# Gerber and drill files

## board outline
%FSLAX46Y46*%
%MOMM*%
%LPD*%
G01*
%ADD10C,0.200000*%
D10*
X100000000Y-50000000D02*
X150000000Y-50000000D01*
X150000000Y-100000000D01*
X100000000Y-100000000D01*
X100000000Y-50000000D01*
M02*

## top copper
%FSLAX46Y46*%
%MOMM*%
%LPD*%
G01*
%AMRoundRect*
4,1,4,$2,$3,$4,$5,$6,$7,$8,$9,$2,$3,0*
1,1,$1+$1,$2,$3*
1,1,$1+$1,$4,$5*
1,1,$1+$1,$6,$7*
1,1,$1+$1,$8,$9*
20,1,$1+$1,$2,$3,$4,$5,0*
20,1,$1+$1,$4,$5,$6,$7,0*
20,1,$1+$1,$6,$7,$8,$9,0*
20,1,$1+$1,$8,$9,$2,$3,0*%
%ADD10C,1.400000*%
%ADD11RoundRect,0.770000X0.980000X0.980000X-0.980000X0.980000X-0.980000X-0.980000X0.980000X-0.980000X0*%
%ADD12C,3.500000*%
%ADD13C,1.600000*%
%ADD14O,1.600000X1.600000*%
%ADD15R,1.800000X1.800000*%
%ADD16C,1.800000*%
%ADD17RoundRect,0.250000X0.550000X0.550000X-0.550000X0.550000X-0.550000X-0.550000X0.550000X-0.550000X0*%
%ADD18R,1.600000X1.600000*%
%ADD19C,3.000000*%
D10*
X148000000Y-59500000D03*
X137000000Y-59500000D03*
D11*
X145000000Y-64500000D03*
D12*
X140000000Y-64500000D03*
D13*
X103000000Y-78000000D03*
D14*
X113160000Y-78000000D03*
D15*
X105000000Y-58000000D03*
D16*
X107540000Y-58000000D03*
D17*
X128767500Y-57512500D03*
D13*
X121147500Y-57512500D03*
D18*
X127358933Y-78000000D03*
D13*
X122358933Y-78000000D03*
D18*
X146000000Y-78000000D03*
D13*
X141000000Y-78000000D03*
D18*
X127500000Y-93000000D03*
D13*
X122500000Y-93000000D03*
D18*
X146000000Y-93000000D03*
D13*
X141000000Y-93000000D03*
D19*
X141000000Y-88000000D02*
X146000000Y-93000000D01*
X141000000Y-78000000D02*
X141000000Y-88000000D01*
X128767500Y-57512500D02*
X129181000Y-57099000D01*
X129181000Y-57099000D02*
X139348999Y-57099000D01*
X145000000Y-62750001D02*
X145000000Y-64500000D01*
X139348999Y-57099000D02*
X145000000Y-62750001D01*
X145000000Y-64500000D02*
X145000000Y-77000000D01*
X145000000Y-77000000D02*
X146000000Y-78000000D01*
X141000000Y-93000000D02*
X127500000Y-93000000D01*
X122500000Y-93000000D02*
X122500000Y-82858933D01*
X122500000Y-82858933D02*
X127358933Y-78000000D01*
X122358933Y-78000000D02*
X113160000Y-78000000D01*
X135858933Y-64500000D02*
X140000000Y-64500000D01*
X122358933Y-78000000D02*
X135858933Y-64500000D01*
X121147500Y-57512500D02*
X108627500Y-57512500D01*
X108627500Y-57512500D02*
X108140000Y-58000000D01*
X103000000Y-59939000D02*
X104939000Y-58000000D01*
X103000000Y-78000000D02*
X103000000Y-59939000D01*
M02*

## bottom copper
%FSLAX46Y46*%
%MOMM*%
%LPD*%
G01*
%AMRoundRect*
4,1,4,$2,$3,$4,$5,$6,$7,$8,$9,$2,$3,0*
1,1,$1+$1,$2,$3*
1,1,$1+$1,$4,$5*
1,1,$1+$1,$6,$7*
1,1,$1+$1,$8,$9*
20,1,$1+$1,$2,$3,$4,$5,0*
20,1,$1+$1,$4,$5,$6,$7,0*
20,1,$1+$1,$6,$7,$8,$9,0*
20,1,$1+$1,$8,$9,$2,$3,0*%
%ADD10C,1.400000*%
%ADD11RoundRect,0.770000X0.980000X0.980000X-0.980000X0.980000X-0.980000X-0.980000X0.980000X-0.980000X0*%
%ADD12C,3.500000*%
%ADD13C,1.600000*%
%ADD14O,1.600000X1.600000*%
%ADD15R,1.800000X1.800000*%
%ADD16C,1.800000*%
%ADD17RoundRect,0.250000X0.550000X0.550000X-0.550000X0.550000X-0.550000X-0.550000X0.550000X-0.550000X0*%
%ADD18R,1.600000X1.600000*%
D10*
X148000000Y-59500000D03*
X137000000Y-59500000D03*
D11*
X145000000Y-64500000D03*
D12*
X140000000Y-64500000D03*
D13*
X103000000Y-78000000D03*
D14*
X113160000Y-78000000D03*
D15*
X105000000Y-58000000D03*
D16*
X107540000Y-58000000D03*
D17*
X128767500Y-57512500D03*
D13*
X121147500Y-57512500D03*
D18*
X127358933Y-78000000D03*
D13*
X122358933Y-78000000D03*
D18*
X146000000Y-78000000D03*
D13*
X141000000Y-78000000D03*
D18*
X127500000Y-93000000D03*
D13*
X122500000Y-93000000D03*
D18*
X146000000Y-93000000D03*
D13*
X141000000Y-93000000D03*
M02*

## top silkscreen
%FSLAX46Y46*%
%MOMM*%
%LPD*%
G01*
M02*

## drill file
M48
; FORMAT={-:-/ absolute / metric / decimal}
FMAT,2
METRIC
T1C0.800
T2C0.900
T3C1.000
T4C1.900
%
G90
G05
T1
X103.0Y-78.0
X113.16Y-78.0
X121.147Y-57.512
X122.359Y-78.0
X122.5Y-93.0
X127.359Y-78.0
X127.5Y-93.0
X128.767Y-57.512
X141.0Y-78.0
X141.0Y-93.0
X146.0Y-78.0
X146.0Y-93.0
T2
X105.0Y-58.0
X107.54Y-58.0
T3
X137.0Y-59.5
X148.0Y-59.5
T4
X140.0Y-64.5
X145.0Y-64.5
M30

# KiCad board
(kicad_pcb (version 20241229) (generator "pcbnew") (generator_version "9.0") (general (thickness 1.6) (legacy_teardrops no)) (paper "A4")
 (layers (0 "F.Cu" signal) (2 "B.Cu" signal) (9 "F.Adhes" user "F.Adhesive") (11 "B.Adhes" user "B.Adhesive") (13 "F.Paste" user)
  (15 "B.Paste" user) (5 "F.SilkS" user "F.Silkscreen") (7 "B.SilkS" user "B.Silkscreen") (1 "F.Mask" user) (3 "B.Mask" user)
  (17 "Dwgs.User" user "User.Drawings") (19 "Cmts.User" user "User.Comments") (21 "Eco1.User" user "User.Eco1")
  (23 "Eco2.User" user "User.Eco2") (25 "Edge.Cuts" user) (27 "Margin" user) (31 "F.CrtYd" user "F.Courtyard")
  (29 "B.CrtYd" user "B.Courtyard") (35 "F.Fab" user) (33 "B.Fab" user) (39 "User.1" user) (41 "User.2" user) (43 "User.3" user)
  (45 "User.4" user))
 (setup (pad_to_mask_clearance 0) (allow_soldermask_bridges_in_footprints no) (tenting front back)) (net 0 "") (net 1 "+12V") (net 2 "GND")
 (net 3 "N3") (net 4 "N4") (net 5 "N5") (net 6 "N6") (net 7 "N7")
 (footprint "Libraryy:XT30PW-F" (layer "B.Cu") (at 145 64.5 180)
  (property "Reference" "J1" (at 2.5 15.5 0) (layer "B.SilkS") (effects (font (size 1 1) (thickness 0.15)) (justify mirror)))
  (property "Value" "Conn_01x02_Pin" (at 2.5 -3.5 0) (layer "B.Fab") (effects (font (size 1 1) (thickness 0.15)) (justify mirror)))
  (pad "" thru_hole circle (at -3 5 90) (size 1.4 1.4) (drill 1) (layers "*.Cu" "*.Mask") (remove_unused_layers no))
  (pad "" thru_hole circle (at 8 5 180) (size 1.4 1.4) (drill 1) (layers "*.Cu" "*.Mask") (remove_unused_layers no))
  (pad "1" thru_hole roundrect (at 0 0 180) (size 3.5 3.5) (drill 1.9) (layers "*.Cu" "*.Mask") (remove_unused_layers no)
   (roundrect_rratio 0.22) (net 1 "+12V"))
  (pad "2" thru_hole circle (at 5 0 180) (size 3.5 3.5) (drill 1.9) (layers "*.Cu" "*.Mask") (remove_unused_layers no) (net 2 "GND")))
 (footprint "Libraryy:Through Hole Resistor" (layer "B.Cu") (at 103 78)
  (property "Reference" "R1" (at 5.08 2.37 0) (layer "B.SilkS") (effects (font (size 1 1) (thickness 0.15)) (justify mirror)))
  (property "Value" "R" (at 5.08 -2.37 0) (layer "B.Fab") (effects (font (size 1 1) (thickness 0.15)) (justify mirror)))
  (pad "1" thru_hole circle (at 0 0) (size 1.6 1.6) (drill 0.8) (layers "*.Cu" "*.Mask") (remove_unused_layers no) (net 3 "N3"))
  (pad "2" thru_hole oval (at 10.16 0) (size 1.6 1.6) (drill 0.8) (layers "*.Cu" "*.Mask") (remove_unused_layers no) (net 2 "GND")))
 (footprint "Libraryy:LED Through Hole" (layer "B.Cu") (at 105 58)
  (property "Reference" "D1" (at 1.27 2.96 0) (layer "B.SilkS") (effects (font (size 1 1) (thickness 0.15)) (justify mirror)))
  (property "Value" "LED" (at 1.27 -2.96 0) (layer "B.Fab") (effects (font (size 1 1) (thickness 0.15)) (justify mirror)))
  (pad "1" thru_hole rect (at 0 0) (size 1.8 1.8) (drill 0.9) (layers "*.Cu" "*.Mask") (remove_unused_layers no) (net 3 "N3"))
  (pad "2" thru_hole circle (at 2.54 0) (size 1.8 1.8) (drill 0.9) (layers "*.Cu" "*.Mask") (remove_unused_layers no) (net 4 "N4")))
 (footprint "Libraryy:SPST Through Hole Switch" (layer "B.Cu") (at 128.7675 57.5125 180)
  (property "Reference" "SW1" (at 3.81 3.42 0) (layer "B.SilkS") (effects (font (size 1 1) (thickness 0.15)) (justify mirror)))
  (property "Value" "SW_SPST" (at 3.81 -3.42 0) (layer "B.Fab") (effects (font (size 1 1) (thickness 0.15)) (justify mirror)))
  (pad "1" thru_hole roundrect (at 0 0 180) (size 1.6 1.6) (drill 0.8) (layers "*.Cu" "*.Mask") (remove_unused_layers no)
   (roundrect_rratio 0.15625) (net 1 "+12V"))
  (pad "2" thru_hole circle (at 7.62 0 180) (size 1.6 1.6) (drill 0.8) (layers "*.Cu" "*.Mask") (remove_unused_layers no) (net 4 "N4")))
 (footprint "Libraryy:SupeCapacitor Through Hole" (layer "B.Cu") (at 127.358933 78 180)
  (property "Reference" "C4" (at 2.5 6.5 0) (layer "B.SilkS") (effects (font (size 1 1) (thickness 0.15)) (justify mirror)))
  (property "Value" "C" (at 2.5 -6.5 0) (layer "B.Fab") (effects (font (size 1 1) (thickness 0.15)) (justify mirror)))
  (pad "1" thru_hole rect (at 0 0 180) (size 1.6 1.6) (drill 0.8) (layers "*.Cu" "*.Mask") (remove_unused_layers no) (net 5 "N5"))
  (pad "2" thru_hole circle (at 5 0 180) (size 1.6 1.6) (drill 0.8) (layers "*.Cu" "*.Mask") (remove_unused_layers no) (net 2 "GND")))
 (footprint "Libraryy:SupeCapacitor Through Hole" (layer "B.Cu") (at 146 78 180)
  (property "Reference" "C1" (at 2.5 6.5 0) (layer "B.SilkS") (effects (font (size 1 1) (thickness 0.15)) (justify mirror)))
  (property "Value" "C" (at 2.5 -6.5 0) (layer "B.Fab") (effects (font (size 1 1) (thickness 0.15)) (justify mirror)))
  (pad "1" thru_hole rect (at 0 0 180) (size 1.6 1.6) (drill 0.8) (layers "*.Cu" "*.Mask") (remove_unused_layers no) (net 1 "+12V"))
  (pad "2" thru_hole circle (at 5 0 180) (size 1.6 1.6) (drill 0.8) (layers "*.Cu" "*.Mask") (remove_unused_layers no) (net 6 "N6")))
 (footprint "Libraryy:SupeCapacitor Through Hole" (layer "B.Cu") (at 127.5 93 180)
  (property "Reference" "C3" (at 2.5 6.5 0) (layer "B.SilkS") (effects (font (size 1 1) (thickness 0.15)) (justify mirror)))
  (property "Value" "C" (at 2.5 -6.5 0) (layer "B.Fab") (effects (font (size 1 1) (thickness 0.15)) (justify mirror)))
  (pad "1" thru_hole rect (at 0 0 180) (size 1.6 1.6) (drill 0.8) (layers "*.Cu" "*.Mask") (remove_unused_layers no) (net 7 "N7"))
  (pad "2" thru_hole circle (at 5 0 180) (size 1.6 1.6) (drill 0.8) (layers "*.Cu" "*.Mask") (remove_unused_layers no) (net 5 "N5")))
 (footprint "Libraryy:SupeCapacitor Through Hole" (layer "B.Cu") (at 146 93 180)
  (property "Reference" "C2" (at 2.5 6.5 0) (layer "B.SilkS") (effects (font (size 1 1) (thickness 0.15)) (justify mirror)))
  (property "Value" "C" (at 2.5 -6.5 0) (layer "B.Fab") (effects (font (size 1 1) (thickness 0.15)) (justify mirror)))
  (pad "1" thru_hole rect (at 0 0 180) (size 1.6 1.6) (drill 0.8) (layers "*.Cu" "*.Mask") (remove_unused_layers no) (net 6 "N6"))
  (pad "2" thru_hole circle (at 5 0 180) (size 1.6 1.6) (drill 0.8) (layers "*.Cu" "*.Mask") (remove_unused_layers no) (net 7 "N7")))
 (gr_rect (start 100 50) (end 150 100) (stroke (width 0.2) (type solid)) (fill no) (layer "Edge.Cuts"))
 (segment (start 141 88) (end 146 93) (width 3) (layer "F.Cu") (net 6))
 (segment (start 141 78) (end 141 88) (width 3) (layer "F.Cu") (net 6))
 (segment (start 128.7675 57.5125) (end 129.181 57.099) (width 3) (layer "F.Cu") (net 1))
 (segment (start 129.181 57.099) (end 139.348999 57.099) (width 3) (layer "F.Cu") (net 1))
 (segment (start 145 62.750001) (end 145 64.5) (width 3) (layer "F.Cu") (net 1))
 (segment (start 139.348999 57.099) (end 145 62.750001) (width 3) (layer "F.Cu") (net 1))
 (segment (start 145 64.5) (end 145 77) (width 3) (layer "F.Cu") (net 1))
 (segment (start 145 77) (end 146 78) (width 3) (layer "F.Cu") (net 1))
 (segment (start 141 93) (end 127.5 93) (width 3) (layer "F.Cu") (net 7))
 (segment (start 122.5 93) (end 122.5 82.858933) (width 3) (layer "F.Cu") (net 5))
 (segment (start 122.5 82.858933) (end 127.358933 78) (width 3) (layer "F.Cu") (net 5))
 (segment (start 122.358933 78) (end 113.16 78) (width 3) (layer "F.Cu") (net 2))
 (segment (start 135.858933 64.5) (end 140 64.5) (width 3) (layer "F.Cu") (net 2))
 (segment (start 122.358933 78) (end 135.858933 64.5) (width 3) (layer "F.Cu") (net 2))
 (segment (start 121.1475 57.5125) (end 108.6275 57.5125) (width 3) (layer "F.Cu") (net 4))
 (segment (start 108.6275 57.5125) (end 108.14 58) (width 3) (layer "F.Cu") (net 4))
 (segment (start 103 59.939) (end 104.939 58) (width 3) (layer "F.Cu") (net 3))
 (segment (start 103 78) (end 103 59.939) (width 3) (layer "F.Cu") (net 3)))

